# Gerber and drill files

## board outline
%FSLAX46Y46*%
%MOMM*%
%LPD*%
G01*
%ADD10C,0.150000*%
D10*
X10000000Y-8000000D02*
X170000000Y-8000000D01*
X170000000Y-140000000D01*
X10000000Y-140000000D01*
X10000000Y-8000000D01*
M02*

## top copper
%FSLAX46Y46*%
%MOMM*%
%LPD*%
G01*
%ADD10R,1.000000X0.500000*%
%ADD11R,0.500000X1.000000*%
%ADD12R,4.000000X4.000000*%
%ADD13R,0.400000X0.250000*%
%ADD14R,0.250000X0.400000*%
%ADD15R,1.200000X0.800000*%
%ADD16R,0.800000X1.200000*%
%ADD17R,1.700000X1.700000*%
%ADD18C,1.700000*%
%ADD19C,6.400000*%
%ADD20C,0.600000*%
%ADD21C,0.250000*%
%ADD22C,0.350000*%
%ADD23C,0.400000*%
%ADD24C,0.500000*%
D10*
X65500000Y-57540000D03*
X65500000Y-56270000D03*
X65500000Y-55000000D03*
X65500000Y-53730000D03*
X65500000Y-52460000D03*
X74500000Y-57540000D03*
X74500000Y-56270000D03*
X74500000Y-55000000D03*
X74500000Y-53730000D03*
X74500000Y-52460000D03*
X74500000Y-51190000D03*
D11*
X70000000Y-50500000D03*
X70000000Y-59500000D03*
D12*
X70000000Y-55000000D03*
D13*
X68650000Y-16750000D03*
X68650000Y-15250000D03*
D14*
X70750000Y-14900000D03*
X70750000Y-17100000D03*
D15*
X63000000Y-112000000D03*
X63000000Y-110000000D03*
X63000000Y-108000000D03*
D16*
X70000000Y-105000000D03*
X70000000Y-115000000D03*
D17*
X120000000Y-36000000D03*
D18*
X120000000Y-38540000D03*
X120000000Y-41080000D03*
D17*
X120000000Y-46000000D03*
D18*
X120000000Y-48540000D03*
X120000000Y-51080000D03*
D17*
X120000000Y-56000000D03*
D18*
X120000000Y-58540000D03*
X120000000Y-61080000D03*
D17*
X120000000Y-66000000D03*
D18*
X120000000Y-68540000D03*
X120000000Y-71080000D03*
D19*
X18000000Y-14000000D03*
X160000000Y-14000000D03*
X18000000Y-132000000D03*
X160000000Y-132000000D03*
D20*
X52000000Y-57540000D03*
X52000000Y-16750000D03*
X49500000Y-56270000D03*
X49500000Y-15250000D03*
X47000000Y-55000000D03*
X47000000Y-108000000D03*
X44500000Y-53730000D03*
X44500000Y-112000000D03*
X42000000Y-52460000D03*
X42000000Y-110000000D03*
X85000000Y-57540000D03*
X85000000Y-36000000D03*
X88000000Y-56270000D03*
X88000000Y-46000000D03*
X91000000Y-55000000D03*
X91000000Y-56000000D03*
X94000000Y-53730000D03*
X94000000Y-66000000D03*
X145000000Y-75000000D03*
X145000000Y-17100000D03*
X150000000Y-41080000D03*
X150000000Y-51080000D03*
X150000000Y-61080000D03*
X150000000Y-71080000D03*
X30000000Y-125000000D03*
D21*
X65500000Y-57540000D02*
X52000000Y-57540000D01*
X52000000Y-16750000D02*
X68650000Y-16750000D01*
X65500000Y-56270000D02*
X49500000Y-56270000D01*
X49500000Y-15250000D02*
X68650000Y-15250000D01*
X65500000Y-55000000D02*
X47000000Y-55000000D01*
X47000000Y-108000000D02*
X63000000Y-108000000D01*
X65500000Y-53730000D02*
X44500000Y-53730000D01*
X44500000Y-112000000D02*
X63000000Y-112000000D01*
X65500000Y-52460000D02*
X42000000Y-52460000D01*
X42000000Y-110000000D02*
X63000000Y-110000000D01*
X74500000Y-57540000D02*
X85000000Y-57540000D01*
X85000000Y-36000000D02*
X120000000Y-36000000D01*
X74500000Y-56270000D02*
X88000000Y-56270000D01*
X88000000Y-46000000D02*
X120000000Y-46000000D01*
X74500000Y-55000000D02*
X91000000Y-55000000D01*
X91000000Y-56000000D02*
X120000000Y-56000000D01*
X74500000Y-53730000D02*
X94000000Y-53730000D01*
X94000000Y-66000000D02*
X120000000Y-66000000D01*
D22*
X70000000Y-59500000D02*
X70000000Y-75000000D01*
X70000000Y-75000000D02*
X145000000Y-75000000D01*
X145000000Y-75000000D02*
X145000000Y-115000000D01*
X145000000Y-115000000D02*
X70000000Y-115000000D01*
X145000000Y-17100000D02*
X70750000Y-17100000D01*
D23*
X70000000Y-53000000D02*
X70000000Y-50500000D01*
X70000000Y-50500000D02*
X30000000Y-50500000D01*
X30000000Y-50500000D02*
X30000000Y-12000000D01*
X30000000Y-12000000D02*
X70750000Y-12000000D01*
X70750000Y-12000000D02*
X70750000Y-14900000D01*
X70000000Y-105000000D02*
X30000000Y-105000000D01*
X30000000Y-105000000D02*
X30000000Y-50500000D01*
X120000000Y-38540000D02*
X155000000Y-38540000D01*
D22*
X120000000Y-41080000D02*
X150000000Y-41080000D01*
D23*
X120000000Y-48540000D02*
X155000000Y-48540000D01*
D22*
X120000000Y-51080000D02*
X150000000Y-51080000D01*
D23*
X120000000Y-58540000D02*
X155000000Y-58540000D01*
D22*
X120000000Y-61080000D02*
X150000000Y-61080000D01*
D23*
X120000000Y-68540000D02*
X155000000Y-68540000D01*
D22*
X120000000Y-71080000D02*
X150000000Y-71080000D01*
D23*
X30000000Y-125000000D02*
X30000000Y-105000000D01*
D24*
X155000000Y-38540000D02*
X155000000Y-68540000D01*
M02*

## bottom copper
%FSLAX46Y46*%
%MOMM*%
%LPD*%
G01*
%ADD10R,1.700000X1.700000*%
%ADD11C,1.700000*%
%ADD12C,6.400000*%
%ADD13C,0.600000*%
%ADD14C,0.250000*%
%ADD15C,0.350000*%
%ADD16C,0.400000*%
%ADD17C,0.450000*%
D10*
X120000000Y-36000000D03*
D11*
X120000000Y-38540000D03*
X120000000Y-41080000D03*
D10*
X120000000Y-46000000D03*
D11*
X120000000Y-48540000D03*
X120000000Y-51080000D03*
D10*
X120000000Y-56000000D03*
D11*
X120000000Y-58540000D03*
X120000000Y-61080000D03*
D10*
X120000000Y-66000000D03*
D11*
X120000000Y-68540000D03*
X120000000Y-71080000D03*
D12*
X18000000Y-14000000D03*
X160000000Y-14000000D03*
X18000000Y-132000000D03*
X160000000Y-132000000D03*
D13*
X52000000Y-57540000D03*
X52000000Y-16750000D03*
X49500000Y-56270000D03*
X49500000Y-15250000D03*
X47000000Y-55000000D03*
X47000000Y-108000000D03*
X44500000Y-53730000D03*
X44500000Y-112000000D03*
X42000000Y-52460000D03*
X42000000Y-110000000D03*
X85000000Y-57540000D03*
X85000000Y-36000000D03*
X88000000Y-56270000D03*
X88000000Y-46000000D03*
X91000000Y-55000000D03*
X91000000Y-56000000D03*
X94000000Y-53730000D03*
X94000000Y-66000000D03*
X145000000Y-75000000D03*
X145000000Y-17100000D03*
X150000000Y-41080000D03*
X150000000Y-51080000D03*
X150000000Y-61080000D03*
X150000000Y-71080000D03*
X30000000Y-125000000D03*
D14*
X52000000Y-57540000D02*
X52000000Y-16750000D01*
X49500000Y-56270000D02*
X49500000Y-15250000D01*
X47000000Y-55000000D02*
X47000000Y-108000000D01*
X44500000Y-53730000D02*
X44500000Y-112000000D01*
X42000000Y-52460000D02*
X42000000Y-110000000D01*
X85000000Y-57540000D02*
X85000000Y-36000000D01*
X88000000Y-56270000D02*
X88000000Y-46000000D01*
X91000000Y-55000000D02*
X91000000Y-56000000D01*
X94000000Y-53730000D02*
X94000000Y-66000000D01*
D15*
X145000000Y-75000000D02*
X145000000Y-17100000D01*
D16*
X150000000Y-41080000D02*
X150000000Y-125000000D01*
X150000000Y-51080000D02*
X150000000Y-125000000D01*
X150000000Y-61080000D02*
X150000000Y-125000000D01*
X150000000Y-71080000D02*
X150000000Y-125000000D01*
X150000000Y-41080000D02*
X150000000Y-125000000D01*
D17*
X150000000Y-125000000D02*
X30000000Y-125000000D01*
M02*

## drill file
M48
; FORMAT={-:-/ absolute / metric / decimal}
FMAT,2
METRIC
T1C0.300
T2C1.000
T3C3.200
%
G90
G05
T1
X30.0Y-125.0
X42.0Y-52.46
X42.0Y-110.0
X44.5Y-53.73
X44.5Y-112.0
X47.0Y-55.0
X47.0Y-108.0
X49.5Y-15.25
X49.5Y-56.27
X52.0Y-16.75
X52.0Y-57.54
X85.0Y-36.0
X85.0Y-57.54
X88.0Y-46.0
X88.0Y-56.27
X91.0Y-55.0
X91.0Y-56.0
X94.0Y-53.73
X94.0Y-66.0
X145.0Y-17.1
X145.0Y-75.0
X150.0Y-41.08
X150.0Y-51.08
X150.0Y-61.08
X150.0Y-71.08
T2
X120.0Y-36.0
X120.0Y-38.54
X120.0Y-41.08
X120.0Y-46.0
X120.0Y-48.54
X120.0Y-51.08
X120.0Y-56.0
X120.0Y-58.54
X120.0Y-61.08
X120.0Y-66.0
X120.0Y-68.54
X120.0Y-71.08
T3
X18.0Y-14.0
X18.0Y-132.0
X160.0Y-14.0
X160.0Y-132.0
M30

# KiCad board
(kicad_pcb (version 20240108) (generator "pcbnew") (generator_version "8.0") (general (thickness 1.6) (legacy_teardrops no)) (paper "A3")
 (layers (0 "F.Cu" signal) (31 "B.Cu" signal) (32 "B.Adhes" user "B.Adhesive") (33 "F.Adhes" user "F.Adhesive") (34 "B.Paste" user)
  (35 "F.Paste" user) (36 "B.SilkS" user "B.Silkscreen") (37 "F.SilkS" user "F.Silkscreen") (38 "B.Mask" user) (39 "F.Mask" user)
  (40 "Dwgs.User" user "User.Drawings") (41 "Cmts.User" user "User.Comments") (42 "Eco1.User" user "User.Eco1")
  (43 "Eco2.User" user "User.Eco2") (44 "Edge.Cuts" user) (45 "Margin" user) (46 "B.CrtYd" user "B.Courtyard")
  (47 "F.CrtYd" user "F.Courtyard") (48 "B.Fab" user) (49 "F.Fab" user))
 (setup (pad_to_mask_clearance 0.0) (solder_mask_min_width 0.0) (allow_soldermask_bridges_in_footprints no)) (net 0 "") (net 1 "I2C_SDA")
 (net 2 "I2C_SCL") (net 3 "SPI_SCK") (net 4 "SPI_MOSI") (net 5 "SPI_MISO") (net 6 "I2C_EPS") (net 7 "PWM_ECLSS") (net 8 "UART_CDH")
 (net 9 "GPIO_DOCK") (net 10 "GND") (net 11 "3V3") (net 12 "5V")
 (gr_rect (start 10 8) (end 170 140) (stroke (width 0.15) (type solid)) (fill none) (layer "Edge.Cuts"))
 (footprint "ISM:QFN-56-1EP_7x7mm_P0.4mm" (layer "F.Cu") (at 70 55)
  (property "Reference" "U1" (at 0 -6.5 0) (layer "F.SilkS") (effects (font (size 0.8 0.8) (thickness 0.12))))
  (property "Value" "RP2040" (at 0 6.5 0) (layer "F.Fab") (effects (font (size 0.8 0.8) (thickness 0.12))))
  (pad "1" smd rect (at -4.5 2.54) (size 1.0 0.5) (layers "F.Cu" "F.Paste" "F.Mask") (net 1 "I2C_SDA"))
  (pad "2" smd rect (at -4.5 1.27) (size 1.0 0.5) (layers "F.Cu" "F.Paste" "F.Mask") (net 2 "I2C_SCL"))
  (pad "3" smd rect (at -4.5 0) (size 1.0 0.5) (layers "F.Cu" "F.Paste" "F.Mask") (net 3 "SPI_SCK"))
  (pad "4" smd rect (at -4.5 -1.27) (size 1.0 0.5) (layers "F.Cu" "F.Paste" "F.Mask") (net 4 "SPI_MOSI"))
  (pad "5" smd rect (at -4.5 -2.54) (size 1.0 0.5) (layers "F.Cu" "F.Paste" "F.Mask") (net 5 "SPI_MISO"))
  (pad "6" smd rect (at 4.5 2.54) (size 1.0 0.5) (layers "F.Cu" "F.Paste" "F.Mask") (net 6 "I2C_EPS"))
  (pad "7" smd rect (at 4.5 1.27) (size 1.0 0.5) (layers "F.Cu" "F.Paste" "F.Mask") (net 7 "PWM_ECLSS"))
  (pad "8" smd rect (at 4.5 0) (size 1.0 0.5) (layers "F.Cu" "F.Paste" "F.Mask") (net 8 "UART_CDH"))
  (pad "9" smd rect (at 4.5 -1.27) (size 1.0 0.5) (layers "F.Cu" "F.Paste" "F.Mask") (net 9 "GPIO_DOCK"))
  (pad "12" smd rect (at 4.5 -2.54) (size 1.0 0.5) (layers "F.Cu" "F.Paste" "F.Mask"))
  (pad "13" smd rect (at 4.5 -3.81) (size 1.0 0.5) (layers "F.Cu" "F.Paste" "F.Mask"))
  (pad "10" smd rect (at 0 -4.5) (size 0.5 1.0) (layers "F.Cu" "F.Paste" "F.Mask") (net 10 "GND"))
  (pad "11" smd rect (at 0 4.5) (size 0.5 1.0) (layers "F.Cu" "F.Paste" "F.Mask") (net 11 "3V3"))
  (pad "EP" smd rect (at 0 0) (size 4 4) (layers "F.Cu" "F.Paste" "F.Mask") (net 10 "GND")))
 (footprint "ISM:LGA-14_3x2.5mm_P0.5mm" (layer "F.Cu") (at 70 16)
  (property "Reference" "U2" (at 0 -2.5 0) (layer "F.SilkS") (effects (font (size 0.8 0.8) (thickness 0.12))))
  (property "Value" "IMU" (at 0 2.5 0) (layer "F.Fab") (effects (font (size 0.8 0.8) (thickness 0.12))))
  (pad "1" smd rect (at -1.35 0.75) (size 0.4 0.25) (layers "F.Cu" "F.Paste" "F.Mask") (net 1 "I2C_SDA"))
  (pad "2" smd rect (at -1.35 -0.75) (size 0.4 0.25) (layers "F.Cu" "F.Paste" "F.Mask") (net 2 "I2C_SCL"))
  (pad "3" smd rect (at 0.75 -1.1) (size 0.25 0.4) (layers "F.Cu" "F.Paste" "F.Mask") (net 10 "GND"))
  (pad "4" smd rect (at 0.75 1.1) (size 0.25 0.4) (layers "F.Cu" "F.Paste" "F.Mask") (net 11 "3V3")))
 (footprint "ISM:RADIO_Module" (layer "F.Cu") (at 70 110)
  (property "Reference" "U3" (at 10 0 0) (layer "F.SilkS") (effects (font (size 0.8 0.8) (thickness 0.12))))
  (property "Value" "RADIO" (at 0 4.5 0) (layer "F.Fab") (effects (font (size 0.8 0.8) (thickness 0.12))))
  (pad "1" smd rect (at -7 2) (size 1.2 0.8) (layers "F.Cu" "F.Paste" "F.Mask") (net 4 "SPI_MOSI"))
  (pad "2" smd rect (at -7 0) (size 1.2 0.8) (layers "F.Cu" "F.Paste" "F.Mask") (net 5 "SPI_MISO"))
  (pad "3" smd rect (at -7 -2) (size 1.2 0.8) (layers "F.Cu" "F.Paste" "F.Mask") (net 3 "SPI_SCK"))
  (pad "4" smd rect (at 0 -5) (size 0.8 1.2) (layers "F.Cu" "F.Paste" "F.Mask") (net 10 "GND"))
  (pad "5" smd rect (at 0 5) (size 0.8 1.2) (layers "F.Cu" "F.Paste" "F.Mask") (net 11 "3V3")))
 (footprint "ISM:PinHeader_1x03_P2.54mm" (layer "F.Cu") (at 120 36)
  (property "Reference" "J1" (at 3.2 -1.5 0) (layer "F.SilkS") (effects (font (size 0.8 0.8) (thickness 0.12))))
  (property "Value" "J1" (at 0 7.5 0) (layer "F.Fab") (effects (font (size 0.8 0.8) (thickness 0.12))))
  (pad "1" thru_hole rect (at 0 0) (size 1.7 1.7) (drill 1.0) (layers "*.Cu" "*.Mask") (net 6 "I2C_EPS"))
  (pad "2" thru_hole circle (at 0 2.54) (size 1.7 1.7) (drill 1.0) (layers "*.Cu" "*.Mask") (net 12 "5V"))
  (pad "3" thru_hole circle (at 0 5.08) (size 1.7 1.7) (drill 1.0) (layers "*.Cu" "*.Mask") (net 10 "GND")))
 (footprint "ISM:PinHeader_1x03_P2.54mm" (layer "F.Cu") (at 120 46)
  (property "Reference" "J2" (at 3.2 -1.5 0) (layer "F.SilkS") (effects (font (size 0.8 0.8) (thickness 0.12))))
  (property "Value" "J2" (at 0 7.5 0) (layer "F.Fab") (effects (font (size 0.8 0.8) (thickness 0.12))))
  (pad "1" thru_hole rect (at 0 0) (size 1.7 1.7) (drill 1.0) (layers "*.Cu" "*.Mask") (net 7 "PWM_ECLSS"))
  (pad "2" thru_hole circle (at 0 2.54) (size 1.7 1.7) (drill 1.0) (layers "*.Cu" "*.Mask") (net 12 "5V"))
  (pad "3" thru_hole circle (at 0 5.08) (size 1.7 1.7) (drill 1.0) (layers "*.Cu" "*.Mask") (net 10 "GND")))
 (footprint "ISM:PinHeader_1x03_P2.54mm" (layer "F.Cu") (at 120 56)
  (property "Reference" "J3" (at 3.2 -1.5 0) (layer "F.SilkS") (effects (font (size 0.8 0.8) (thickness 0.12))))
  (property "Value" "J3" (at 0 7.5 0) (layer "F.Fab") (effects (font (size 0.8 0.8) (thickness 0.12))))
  (pad "1" thru_hole rect (at 0 0) (size 1.7 1.7) (drill 1.0) (layers "*.Cu" "*.Mask") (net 8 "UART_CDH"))
  (pad "2" thru_hole circle (at 0 2.54) (size 1.7 1.7) (drill 1.0) (layers "*.Cu" "*.Mask") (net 12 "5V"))
  (pad "3" thru_hole circle (at 0 5.08) (size 1.7 1.7) (drill 1.0) (layers "*.Cu" "*.Mask") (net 10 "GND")))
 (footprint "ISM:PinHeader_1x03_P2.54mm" (layer "F.Cu") (at 120 66)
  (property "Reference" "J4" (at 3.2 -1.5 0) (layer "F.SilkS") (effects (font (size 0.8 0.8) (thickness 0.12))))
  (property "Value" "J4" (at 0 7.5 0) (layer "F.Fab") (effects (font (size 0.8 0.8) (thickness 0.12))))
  (pad "1" thru_hole rect (at 0 0) (size 1.7 1.7) (drill 1.0) (layers "*.Cu" "*.Mask") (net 9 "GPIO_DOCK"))
  (pad "2" thru_hole circle (at 0 2.54) (size 1.7 1.7) (drill 1.0) (layers "*.Cu" "*.Mask") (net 12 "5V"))
  (pad "3" thru_hole circle (at 0 5.08) (size 1.7 1.7) (drill 1.0) (layers "*.Cu" "*.Mask") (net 10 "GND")))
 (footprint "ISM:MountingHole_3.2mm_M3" (layer "F.Cu") (at 18 14)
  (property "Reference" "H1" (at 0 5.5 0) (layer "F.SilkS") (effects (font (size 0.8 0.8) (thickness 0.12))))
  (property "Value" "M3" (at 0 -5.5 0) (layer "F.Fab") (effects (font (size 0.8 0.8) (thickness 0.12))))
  (pad "" thru_hole circle (at 0 0) (size 6.4 6.4) (drill 3.2) (layers "*.Cu" "*.Mask")))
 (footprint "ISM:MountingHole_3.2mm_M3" (layer "F.Cu") (at 160 14)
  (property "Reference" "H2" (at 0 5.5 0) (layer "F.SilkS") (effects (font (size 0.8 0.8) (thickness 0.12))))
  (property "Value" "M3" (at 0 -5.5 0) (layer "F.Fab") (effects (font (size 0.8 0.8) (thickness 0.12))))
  (pad "" thru_hole circle (at 0 0) (size 6.4 6.4) (drill 3.2) (layers "*.Cu" "*.Mask")))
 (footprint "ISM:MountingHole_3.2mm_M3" (layer "F.Cu") (at 18 132)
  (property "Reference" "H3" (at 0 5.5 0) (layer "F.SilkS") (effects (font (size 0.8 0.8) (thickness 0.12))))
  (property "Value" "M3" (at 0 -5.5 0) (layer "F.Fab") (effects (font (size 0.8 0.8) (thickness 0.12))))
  (pad "" thru_hole circle (at 0 0) (size 6.4 6.4) (drill 3.2) (layers "*.Cu" "*.Mask")))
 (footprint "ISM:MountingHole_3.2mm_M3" (layer "F.Cu") (at 160 132)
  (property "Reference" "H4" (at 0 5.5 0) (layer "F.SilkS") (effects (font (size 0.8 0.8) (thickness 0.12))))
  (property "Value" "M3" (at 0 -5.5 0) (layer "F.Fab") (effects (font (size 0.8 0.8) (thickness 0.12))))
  (pad "" thru_hole circle (at 0 0) (size 6.4 6.4) (drill 3.2) (layers "*.Cu" "*.Mask")))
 (segment (start 65.5 57.54) (end 52.0 57.54) (width 0.25) (layer "F.Cu") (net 1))
 (segment (start 52.0 57.54) (end 52.0 16.75) (width 0.25) (layer "B.Cu") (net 1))
 (segment (start 52.0 16.75) (end 68.65 16.75) (width 0.25) (layer "F.Cu") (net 1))
 (segment (start 65.5 56.27) (end 49.5 56.27) (width 0.25) (layer "F.Cu") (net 2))
 (segment (start 49.5 56.27) (end 49.5 15.25) (width 0.25) (layer "B.Cu") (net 2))
 (segment (start 49.5 15.25) (end 68.65 15.25) (width 0.25) (layer "F.Cu") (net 2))
 (segment (start 65.5 55) (end 47.0 55) (width 0.25) (layer "F.Cu") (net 3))
 (segment (start 47.0 55) (end 47.0 108) (width 0.25) (layer "B.Cu") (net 3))
 (segment (start 47.0 108) (end 63 108) (width 0.25) (layer "F.Cu") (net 3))
 (segment (start 65.5 53.73) (end 44.5 53.73) (width 0.25) (layer "F.Cu") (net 4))
 (segment (start 44.5 53.73) (end 44.5 112) (width 0.25) (layer "B.Cu") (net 4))
 (segment (start 44.5 112) (end 63 112) (width 0.25) (layer "F.Cu") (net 4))
 (segment (start 65.5 52.46) (end 42.0 52.46) (width 0.25) (layer "F.Cu") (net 5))
 (segment (start 42.0 52.46) (end 42.0 110) (width 0.25) (layer "B.Cu") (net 5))
 (segment (start 42.0 110) (end 63 110) (width 0.25) (layer "F.Cu") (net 5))
 (segment (start 74.5 57.54) (end 85 57.54) (width 0.25) (layer "F.Cu") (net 6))
 (segment (start 85 57.54) (end 85 36) (width 0.25) (layer "B.Cu") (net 6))
 (segment (start 85 36) (end 120 36) (width 0.25) (layer "F.Cu") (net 6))
 (segment (start 74.5 56.27) (end 88 56.27) (width 0.25) (layer "F.Cu") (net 7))
 (segment (start 88 56.27) (end 88 46) (width 0.25) (layer "B.Cu") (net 7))
 (segment (start 88 46) (end 120 46) (width 0.25) (layer "F.Cu") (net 7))
 (segment (start 74.5 55) (end 91 55) (width 0.25) (layer "F.Cu") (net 8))
 (segment (start 91 55) (end 91 56) (width 0.25) (layer "B.Cu") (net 8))
 (segment (start 91 56) (end 120 56) (width 0.25) (layer "F.Cu") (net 8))
 (segment (start 74.5 53.73) (end 94 53.73) (width 0.25) (layer "F.Cu") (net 9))
 (segment (start 94 53.73) (end 94 66) (width 0.25) (layer "B.Cu") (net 9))
 (segment (start 94 66) (end 120 66) (width 0.25) (layer "F.Cu") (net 9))
 (segment (start 70 59.5) (end 70 75) (width 0.35) (layer "F.Cu") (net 11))
 (segment (start 70 75) (end 145 75) (width 0.35) (layer "F.Cu") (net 11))
 (segment (start 145 75) (end 145 115) (width 0.35) (layer "F.Cu") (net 11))
 (segment (start 145 115) (end 70 115) (width 0.35) (layer "F.Cu") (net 11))
 (segment (start 145 75) (end 145 17.1) (width 0.35) (layer "B.Cu") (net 11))
 (segment (start 145 17.1) (end 70.75 17.1) (width 0.35) (layer "F.Cu") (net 11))
 (segment (start 70 53) (end 70 50.5) (width 0.4) (layer "F.Cu") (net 10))
 (segment (start 70 50.5) (end 30 50.5) (width 0.4) (layer "F.Cu") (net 10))
 (segment (start 30 50.5) (end 30 12) (width 0.4) (layer "F.Cu") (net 10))
 (segment (start 30 12) (end 70.75 12) (width 0.4) (layer "F.Cu") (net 10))
 (segment (start 70.75 12) (end 70.75 14.9) (width 0.4) (layer "F.Cu") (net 10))
 (segment (start 70 105) (end 30 105) (width 0.4) (layer "F.Cu") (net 10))
 (segment (start 30 105) (end 30 50.5) (width 0.4) (layer "F.Cu") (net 10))
 (segment (start 120 38.54) (end 155 38.54) (width 0.4) (layer "F.Cu") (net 12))
 (segment (start 120 41.08) (end 150 41.08) (width 0.35) (layer "F.Cu") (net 10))
 (segment (start 150 41.08) (end 150 125) (width 0.4) (layer "B.Cu") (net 10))
 (segment (start 120 48.54) (end 155 48.54) (width 0.4) (layer "F.Cu") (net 12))
 (segment (start 120 51.08) (end 150 51.08) (width 0.35) (layer "F.Cu") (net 10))
 (segment (start 150 51.08) (end 150 125) (width 0.4) (layer "B.Cu") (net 10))
 (segment (start 120 58.54) (end 155 58.54) (width 0.4) (layer "F.Cu") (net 12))
 (segment (start 120 61.08) (end 150 61.08) (width 0.35) (layer "F.Cu") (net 10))
 (segment (start 150 61.08) (end 150 125) (width 0.4) (layer "B.Cu") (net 10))
 (segment (start 120 68.54) (end 155 68.54) (width 0.4) (layer "F.Cu") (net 12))
 (segment (start 120 71.08) (end 150 71.08) (width 0.35) (layer "F.Cu") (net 10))
 (segment (start 150 71.08) (end 150 125) (width 0.4) (layer "B.Cu") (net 10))
 (segment (start 150 41.08) (end 150 125) (width 0.4) (layer "B.Cu") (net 10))
 (segment (start 150 125) (end 30 125) (width 0.45) (layer "B.Cu") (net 10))
 (segment (start 30 125) (end 30 105) (width 0.4) (layer "F.Cu") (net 10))
 (segment (start 155 38.54) (end 155 68.54) (width 0.5) (layer "F.Cu") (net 12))
 (via (at 52.0 57.54) (size 0.6) (drill 0.3) (layers "F.Cu" "B.Cu") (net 1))
 (via (at 52.0 16.75) (size 0.6) (drill 0.3) (layers "F.Cu" "B.Cu") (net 1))
 (via (at 49.5 56.27) (size 0.6) (drill 0.3) (layers "F.Cu" "B.Cu") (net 2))
 (via (at 49.5 15.25) (size 0.6) (drill 0.3) (layers "F.Cu" "B.Cu") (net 2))
 (via (at 47.0 55) (size 0.6) (drill 0.3) (layers "F.Cu" "B.Cu") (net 3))
 (via (at 47.0 108) (size 0.6) (drill 0.3) (layers "F.Cu" "B.Cu") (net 3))
 (via (at 44.5 53.73) (size 0.6) (drill 0.3) (layers "F.Cu" "B.Cu") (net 4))
 (via (at 44.5 112) (size 0.6) (drill 0.3) (layers "F.Cu" "B.Cu") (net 4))
 (via (at 42.0 52.46) (size 0.6) (drill 0.3) (layers "F.Cu" "B.Cu") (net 5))
 (via (at 42.0 110) (size 0.6) (drill 0.3) (layers "F.Cu" "B.Cu") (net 5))
 (via (at 85 57.54) (size 0.6) (drill 0.3) (layers "F.Cu" "B.Cu") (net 6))
 (via (at 85 36) (size 0.6) (drill 0.3) (layers "F.Cu" "B.Cu") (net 6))
 (via (at 88 56.27) (size 0.6) (drill 0.3) (layers "F.Cu" "B.Cu") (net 7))
 (via (at 88 46) (size 0.6) (drill 0.3) (layers "F.Cu" "B.Cu") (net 7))
 (via (at 91 55) (size 0.6) (drill 0.3) (layers "F.Cu" "B.Cu") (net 8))
 (via (at 91 56) (size 0.6) (drill 0.3) (layers "F.Cu" "B.Cu") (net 8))
 (via (at 94 53.73) (size 0.6) (drill 0.3) (layers "F.Cu" "B.Cu") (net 9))
 (via (at 94 66) (size 0.6) (drill 0.3) (layers "F.Cu" "B.Cu") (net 9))
 (via (at 145 75) (size 0.6) (drill 0.3) (layers "F.Cu" "B.Cu") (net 11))
 (via (at 145 17.1) (size 0.6) (drill 0.3) (layers "F.Cu" "B.Cu") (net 11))
 (via (at 150 41.08) (size 0.6) (drill 0.3) (layers "F.Cu" "B.Cu") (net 10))
 (via (at 150 51.08) (size 0.6) (drill 0.3) (layers "F.Cu" "B.Cu") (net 10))
 (via (at 150 61.08) (size 0.6) (drill 0.3) (layers "F.Cu" "B.Cu") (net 10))
 (via (at 150 71.08) (size 0.6) (drill 0.3) (layers "F.Cu" "B.Cu") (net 10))
 (via (at 30 125) (size 0.6) (drill 0.3) (layers "F.Cu" "B.Cu") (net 10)))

